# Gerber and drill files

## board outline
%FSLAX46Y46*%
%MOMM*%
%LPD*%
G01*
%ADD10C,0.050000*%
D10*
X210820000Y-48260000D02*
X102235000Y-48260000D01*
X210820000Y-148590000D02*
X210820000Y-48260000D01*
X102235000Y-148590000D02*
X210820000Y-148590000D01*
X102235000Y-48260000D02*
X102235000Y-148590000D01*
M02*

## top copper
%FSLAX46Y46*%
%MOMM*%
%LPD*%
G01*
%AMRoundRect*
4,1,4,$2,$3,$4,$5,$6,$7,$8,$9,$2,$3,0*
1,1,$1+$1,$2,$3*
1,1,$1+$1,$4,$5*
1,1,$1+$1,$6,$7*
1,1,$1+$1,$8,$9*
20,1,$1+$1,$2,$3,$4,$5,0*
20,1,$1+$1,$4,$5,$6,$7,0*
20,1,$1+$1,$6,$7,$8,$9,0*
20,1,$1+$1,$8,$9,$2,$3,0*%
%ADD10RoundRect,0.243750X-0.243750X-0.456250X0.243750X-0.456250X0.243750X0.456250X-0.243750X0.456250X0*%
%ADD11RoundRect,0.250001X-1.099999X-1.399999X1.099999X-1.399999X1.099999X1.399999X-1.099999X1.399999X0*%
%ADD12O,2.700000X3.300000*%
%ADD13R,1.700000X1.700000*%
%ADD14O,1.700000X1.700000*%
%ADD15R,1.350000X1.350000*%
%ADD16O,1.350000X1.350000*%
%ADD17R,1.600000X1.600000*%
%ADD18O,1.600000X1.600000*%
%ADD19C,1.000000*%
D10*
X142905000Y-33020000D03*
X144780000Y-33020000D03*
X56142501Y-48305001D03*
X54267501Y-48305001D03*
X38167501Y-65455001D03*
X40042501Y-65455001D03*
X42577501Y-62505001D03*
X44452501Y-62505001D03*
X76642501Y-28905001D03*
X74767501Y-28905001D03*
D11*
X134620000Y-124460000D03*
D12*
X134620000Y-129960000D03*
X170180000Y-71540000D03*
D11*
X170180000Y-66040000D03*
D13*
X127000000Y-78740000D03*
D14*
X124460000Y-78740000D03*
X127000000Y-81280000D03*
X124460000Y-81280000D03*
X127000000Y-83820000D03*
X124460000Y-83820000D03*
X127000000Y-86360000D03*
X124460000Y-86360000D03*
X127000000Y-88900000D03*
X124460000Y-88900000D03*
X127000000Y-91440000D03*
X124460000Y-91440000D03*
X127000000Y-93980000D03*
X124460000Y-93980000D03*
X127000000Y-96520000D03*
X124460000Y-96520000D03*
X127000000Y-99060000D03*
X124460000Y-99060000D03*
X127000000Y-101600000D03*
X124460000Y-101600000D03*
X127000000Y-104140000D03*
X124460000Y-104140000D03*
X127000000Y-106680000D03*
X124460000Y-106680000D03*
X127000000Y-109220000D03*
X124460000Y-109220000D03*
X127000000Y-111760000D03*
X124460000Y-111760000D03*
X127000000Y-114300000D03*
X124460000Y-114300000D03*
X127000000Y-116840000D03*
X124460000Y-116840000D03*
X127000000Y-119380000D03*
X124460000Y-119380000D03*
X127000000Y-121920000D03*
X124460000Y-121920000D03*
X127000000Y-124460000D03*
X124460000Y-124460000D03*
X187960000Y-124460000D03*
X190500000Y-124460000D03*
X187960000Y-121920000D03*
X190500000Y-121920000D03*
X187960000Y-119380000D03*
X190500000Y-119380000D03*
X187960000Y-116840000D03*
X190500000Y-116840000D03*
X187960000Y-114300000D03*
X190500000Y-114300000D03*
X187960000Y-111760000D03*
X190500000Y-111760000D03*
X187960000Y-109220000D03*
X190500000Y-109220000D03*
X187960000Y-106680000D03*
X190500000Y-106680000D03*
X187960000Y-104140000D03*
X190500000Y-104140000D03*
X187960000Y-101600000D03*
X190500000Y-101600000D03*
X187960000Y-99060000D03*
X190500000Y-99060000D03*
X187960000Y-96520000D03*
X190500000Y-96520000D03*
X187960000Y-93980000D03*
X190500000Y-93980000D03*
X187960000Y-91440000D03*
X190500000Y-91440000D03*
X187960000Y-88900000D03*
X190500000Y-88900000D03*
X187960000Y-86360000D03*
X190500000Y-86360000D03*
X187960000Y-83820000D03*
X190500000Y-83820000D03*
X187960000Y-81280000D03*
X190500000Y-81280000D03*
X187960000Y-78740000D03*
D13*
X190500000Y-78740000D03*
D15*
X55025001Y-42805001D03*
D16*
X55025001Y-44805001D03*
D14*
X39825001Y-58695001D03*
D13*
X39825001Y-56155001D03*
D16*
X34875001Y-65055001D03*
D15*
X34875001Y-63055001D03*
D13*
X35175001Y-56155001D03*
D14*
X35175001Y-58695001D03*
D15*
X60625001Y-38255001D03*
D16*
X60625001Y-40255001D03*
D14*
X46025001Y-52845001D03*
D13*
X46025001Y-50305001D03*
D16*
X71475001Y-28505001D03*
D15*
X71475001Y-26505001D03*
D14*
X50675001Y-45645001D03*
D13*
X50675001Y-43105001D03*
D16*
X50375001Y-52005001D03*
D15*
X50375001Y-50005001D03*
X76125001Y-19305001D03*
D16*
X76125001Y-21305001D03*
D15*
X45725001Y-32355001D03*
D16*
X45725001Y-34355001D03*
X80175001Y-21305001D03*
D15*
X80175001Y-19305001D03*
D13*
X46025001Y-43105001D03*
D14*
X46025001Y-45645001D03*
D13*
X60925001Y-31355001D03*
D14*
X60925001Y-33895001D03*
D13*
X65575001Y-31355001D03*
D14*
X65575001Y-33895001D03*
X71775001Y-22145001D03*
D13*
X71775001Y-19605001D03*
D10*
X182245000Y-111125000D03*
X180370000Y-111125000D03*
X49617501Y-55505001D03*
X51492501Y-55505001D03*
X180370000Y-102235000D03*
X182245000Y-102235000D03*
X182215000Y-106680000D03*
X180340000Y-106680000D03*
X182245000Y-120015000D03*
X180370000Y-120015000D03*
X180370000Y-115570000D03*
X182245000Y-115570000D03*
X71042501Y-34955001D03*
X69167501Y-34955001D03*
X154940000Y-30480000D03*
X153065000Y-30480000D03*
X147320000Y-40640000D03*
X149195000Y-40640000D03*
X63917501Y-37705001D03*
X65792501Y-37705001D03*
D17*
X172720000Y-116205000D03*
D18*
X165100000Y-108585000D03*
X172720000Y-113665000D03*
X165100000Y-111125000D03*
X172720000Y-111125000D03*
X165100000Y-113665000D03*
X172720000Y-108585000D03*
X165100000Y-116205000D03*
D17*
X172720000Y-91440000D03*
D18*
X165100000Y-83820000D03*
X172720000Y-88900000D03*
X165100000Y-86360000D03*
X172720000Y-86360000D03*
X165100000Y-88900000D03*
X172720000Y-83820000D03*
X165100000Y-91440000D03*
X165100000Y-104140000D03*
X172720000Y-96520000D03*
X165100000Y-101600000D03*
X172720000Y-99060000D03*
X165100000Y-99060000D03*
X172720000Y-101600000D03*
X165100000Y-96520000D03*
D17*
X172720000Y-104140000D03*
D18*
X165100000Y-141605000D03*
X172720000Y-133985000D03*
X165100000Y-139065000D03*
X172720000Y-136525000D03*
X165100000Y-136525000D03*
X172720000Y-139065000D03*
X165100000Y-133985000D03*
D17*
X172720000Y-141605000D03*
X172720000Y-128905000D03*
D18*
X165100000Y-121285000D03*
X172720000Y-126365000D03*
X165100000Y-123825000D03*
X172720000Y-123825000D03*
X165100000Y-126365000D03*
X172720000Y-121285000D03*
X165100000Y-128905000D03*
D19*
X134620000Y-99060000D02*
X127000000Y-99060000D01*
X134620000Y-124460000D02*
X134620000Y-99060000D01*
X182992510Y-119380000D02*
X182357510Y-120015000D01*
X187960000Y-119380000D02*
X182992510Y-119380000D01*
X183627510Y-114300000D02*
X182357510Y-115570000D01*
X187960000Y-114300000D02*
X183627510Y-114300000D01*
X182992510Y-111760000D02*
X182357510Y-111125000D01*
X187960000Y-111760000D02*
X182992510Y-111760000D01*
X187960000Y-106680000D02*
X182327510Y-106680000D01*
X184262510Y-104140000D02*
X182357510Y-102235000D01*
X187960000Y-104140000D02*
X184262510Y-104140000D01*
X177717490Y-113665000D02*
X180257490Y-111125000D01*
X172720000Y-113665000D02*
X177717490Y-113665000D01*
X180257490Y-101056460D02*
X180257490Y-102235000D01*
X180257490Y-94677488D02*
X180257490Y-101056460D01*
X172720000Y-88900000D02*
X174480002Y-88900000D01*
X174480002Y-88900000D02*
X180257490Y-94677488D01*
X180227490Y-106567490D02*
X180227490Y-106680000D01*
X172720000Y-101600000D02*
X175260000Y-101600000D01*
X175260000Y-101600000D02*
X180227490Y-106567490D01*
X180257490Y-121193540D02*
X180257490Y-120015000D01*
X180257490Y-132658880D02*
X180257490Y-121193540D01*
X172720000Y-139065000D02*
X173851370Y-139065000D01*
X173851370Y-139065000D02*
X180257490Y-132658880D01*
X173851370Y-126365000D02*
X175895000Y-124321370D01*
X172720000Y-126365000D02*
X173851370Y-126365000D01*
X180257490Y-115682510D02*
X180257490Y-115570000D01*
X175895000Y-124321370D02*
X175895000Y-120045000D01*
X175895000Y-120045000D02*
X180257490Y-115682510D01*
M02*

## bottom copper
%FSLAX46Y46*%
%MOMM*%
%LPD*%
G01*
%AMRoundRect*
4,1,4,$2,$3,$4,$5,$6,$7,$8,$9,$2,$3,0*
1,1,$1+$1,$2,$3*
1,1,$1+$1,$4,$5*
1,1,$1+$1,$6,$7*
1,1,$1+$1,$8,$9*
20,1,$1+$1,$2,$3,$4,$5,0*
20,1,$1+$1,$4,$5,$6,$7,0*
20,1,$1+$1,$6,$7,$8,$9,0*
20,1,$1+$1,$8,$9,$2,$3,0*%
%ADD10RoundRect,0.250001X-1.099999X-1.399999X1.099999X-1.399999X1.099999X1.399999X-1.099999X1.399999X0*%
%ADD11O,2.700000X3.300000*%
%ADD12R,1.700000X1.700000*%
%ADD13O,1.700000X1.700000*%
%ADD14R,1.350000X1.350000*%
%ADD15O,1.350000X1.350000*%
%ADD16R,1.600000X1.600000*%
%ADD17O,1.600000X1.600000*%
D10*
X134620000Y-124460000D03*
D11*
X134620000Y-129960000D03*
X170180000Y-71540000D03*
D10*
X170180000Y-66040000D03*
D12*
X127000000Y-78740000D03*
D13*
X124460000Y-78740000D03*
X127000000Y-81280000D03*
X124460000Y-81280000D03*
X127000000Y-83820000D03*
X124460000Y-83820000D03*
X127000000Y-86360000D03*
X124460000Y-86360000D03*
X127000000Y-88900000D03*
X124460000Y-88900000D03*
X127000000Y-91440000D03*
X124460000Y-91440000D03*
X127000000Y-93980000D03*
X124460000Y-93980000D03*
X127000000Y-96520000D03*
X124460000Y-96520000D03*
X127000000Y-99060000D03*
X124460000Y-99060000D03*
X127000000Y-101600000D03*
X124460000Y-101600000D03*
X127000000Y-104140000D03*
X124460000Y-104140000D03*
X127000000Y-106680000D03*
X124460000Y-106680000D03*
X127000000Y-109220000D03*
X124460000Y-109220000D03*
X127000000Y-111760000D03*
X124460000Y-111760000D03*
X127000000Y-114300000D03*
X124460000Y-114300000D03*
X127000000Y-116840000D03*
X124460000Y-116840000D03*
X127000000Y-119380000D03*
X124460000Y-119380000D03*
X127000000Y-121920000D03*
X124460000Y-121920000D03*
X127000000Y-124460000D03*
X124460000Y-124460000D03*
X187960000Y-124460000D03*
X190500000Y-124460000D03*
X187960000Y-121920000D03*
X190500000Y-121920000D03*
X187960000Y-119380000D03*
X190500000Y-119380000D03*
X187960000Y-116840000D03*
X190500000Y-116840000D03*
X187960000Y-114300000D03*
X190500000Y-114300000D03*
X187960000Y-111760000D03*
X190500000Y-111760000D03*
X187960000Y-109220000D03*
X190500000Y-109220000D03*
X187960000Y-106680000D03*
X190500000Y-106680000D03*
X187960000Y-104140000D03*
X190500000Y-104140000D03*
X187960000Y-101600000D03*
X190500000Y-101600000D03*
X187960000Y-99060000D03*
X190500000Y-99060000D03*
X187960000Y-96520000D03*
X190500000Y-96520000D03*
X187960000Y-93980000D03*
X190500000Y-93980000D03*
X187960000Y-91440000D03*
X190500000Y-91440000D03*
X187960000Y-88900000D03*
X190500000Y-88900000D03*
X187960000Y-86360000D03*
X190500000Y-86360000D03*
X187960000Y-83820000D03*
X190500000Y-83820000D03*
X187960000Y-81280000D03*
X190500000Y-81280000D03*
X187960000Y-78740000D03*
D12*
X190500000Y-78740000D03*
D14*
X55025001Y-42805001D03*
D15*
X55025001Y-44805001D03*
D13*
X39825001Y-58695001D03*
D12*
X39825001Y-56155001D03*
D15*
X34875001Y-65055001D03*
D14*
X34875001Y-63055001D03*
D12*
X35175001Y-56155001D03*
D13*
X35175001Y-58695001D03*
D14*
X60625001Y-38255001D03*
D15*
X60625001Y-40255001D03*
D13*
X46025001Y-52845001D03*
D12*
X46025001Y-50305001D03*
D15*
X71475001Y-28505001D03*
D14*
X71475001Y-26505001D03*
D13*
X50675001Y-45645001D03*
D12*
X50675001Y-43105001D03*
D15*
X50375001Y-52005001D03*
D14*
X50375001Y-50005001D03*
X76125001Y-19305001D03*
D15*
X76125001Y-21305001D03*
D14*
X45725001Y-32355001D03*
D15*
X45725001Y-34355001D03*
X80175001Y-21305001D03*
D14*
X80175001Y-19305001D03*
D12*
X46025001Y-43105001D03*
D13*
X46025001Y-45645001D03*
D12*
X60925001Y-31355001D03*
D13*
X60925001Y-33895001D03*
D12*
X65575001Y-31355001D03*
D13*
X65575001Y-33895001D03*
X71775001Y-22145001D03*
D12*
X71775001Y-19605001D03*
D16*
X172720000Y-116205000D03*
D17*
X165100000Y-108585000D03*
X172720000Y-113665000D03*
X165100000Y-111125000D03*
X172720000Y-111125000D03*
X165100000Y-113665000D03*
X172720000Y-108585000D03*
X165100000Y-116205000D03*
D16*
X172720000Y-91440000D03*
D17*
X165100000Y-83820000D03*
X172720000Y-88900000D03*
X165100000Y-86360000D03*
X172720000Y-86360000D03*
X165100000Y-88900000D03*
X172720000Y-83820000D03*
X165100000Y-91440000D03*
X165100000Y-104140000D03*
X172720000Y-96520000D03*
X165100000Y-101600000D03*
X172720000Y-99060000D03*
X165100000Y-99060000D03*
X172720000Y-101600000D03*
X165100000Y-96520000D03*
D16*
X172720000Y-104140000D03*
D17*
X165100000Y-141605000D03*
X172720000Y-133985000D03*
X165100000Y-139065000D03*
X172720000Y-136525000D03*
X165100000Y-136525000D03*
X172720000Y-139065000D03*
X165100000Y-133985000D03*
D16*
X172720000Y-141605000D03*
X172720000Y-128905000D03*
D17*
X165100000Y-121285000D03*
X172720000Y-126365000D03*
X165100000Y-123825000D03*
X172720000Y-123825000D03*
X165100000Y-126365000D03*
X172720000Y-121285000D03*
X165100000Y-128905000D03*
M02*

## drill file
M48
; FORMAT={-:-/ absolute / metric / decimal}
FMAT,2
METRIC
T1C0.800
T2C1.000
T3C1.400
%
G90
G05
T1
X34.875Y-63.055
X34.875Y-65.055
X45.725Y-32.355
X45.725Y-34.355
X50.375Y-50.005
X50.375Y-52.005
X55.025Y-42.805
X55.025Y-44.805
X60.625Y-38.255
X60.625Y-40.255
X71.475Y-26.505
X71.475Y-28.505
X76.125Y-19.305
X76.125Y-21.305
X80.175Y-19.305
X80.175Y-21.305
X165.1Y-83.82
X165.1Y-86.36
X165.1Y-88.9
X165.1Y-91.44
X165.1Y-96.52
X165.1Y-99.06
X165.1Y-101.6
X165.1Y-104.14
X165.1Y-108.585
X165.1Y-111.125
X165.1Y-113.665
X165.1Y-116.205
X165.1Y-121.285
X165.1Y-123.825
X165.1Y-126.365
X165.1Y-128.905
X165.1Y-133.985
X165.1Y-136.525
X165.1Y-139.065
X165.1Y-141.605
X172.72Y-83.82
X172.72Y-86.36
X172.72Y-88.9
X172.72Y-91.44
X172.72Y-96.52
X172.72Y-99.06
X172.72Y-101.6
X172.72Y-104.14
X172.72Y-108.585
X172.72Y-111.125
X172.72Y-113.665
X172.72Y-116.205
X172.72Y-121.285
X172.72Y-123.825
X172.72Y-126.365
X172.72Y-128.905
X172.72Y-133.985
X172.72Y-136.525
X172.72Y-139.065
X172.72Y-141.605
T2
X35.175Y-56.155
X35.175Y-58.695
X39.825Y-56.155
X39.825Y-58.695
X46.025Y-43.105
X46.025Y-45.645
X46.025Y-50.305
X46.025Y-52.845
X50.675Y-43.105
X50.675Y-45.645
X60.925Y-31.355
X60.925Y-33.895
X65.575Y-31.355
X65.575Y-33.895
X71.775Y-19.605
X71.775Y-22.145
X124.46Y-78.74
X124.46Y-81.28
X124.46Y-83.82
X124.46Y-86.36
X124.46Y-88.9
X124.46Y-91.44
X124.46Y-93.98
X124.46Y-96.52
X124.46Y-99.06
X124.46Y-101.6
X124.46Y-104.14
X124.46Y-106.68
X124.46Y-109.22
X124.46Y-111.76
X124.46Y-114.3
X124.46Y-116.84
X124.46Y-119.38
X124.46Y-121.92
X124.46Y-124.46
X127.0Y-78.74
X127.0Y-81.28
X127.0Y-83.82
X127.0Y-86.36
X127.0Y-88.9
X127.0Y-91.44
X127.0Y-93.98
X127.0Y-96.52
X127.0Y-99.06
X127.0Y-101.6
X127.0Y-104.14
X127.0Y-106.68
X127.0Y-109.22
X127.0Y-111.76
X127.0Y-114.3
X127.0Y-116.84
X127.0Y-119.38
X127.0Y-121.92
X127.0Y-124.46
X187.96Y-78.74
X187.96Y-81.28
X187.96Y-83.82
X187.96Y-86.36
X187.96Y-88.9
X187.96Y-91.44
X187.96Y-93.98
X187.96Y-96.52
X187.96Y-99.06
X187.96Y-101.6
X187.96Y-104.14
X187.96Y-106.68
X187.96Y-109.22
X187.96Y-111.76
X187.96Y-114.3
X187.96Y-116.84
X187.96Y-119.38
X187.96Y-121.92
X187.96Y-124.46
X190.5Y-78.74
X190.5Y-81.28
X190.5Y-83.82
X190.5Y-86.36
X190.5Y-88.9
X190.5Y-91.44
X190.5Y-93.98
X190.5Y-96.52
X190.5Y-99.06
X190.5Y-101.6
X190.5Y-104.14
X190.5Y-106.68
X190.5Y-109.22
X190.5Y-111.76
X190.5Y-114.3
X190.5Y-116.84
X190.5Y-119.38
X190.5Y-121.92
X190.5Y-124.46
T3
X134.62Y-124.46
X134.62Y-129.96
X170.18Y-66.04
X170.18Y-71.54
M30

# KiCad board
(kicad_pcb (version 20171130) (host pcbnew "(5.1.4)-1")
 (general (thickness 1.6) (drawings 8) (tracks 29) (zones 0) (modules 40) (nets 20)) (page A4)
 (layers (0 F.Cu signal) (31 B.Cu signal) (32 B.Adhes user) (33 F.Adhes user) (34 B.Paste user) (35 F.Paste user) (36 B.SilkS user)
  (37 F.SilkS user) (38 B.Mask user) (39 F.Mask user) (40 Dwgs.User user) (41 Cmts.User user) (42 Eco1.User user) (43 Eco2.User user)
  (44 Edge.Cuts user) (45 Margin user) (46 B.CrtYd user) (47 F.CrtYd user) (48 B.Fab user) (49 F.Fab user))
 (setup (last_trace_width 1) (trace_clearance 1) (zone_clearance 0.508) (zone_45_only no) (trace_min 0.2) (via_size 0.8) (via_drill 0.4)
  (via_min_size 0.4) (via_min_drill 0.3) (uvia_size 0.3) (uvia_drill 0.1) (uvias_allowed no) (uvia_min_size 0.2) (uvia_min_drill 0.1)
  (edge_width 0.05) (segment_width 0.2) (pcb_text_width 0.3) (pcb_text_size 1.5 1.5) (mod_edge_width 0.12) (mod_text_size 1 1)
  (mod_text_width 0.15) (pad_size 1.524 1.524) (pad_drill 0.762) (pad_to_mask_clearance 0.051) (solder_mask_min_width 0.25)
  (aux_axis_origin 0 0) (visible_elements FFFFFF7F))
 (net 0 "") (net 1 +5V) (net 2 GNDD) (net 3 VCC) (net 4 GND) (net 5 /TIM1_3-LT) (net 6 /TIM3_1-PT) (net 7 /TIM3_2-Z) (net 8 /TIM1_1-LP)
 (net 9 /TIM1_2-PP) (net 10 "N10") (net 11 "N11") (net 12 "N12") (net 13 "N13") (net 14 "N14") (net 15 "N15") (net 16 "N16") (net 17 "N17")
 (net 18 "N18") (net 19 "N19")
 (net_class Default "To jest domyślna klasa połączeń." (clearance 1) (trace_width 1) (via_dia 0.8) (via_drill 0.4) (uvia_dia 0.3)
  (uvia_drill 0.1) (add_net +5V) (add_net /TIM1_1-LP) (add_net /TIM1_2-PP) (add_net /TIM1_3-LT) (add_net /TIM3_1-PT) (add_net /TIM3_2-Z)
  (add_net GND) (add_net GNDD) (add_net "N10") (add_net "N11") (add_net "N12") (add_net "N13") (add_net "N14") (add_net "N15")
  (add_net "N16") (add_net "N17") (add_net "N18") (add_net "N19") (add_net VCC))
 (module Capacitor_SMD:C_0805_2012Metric (layer F.Cu) (at 143.8425 33.02)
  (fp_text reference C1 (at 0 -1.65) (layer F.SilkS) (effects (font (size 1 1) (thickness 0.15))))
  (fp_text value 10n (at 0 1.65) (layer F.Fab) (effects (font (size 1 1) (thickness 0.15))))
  (pad 1 smd roundrect (at -0.9375 0) (size 0.975 1.4) (layers F.Cu F.Paste F.Mask) (roundrect_rratio 0.25) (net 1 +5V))
  (pad 2 smd roundrect (at 0.9375 0) (size 0.975 1.4) (layers F.Cu F.Paste F.Mask) (roundrect_rratio 0.25) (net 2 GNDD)))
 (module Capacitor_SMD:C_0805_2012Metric (layer F.Cu) (at 55.205001 48.305001)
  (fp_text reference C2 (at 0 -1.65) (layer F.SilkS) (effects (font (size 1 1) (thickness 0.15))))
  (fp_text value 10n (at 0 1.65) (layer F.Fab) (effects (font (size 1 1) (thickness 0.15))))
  (pad 2 smd roundrect (at 0.9375 0) (size 0.975 1.4) (layers F.Cu F.Paste F.Mask) (roundrect_rratio 0.25) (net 2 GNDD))
  (pad 1 smd roundrect (at -0.9375 0) (size 0.975 1.4) (layers F.Cu F.Paste F.Mask) (roundrect_rratio 0.25) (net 1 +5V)))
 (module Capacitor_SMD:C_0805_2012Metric (layer F.Cu) (at 39.105001 65.455001)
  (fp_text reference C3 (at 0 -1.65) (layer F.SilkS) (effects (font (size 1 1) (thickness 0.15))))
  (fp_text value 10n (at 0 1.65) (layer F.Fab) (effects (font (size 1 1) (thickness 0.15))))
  (pad 1 smd roundrect (at -0.9375 0) (size 0.975 1.4) (layers F.Cu F.Paste F.Mask) (roundrect_rratio 0.25) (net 1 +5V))
  (pad 2 smd roundrect (at 0.9375 0) (size 0.975 1.4) (layers F.Cu F.Paste F.Mask) (roundrect_rratio 0.25) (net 2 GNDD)))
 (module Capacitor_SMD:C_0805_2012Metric (layer F.Cu) (at 43.515001 62.505001)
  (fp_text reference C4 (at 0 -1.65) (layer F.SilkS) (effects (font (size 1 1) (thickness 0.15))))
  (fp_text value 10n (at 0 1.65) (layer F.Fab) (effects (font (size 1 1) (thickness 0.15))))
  (pad 1 smd roundrect (at -0.9375 0) (size 0.975 1.4) (layers F.Cu F.Paste F.Mask) (roundrect_rratio 0.25) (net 1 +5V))
  (pad 2 smd roundrect (at 0.9375 0) (size 0.975 1.4) (layers F.Cu F.Paste F.Mask) (roundrect_rratio 0.25) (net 2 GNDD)))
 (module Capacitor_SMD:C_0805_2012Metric (layer F.Cu) (at 75.705001 28.905001)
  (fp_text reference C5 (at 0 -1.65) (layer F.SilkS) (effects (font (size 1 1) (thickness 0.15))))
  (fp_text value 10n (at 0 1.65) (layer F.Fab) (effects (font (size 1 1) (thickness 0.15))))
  (pad 2 smd roundrect (at 0.9375 0) (size 0.975 1.4) (layers F.Cu F.Paste F.Mask) (roundrect_rratio 0.25) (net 2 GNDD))
  (pad 1 smd roundrect (at -0.9375 0) (size 0.975 1.4) (layers F.Cu F.Paste F.Mask) (roundrect_rratio 0.25) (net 1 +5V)))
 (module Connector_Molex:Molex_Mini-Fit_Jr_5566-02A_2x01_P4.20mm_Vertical (layer F.Cu) (at 134.62 124.46)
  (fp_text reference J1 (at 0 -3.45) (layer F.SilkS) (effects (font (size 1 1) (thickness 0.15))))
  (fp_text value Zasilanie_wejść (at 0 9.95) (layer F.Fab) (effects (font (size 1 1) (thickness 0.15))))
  (pad 1 thru_hole roundrect (at 0 0) (size 2.7 3.3) (drill 1.4) (layers *.Cu *.Mask) (roundrect_rratio 0.09259299999999999) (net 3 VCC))
  (pad 2 thru_hole oval (at 0 5.5) (size 2.7 3.3) (drill 1.4) (layers *.Cu *.Mask) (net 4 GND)))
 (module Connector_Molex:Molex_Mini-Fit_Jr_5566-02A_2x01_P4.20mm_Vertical (layer F.Cu) (at 170.18 66.04)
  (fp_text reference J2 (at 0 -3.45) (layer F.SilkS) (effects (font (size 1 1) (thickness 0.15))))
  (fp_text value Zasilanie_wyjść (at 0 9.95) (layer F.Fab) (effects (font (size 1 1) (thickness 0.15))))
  (pad 2 thru_hole oval (at 0 5.5) (size 2.7 3.3) (drill 1.4) (layers *.Cu *.Mask) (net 2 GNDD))
  (pad 1 thru_hole roundrect (at 0 0) (size 2.7 3.3) (drill 1.4) (layers *.Cu *.Mask) (roundrect_rratio 0.09259299999999999) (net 1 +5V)))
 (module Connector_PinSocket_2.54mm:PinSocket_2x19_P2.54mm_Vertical (layer F.Cu) (at 127 78.74)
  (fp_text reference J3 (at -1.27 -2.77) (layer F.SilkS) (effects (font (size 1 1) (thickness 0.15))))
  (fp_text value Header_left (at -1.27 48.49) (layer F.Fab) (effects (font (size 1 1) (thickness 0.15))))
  (pad 1 thru_hole rect (at 0 0) (size 1.7 1.7) (drill 1) (layers *.Cu *.Mask))
  (pad 2 thru_hole oval (at -2.54 0) (size 1.7 1.7) (drill 1) (layers *.Cu *.Mask))
  (pad 3 thru_hole oval (at 0 2.54) (size 1.7 1.7) (drill 1) (layers *.Cu *.Mask))
  (pad 4 thru_hole oval (at -2.54 2.54) (size 1.7 1.7) (drill 1) (layers *.Cu *.Mask))
  (pad 5 thru_hole oval (at 0 5.08) (size 1.7 1.7) (drill 1) (layers *.Cu *.Mask))
  (pad 6 thru_hole oval (at -2.54 5.08) (size 1.7 1.7) (drill 1) (layers *.Cu *.Mask))
  (pad 7 thru_hole oval (at 0 7.62) (size 1.7 1.7) (drill 1) (layers *.Cu *.Mask))
  (pad 8 thru_hole oval (at -2.54 7.62) (size 1.7 1.7) (drill 1) (layers *.Cu *.Mask))
  (pad 9 thru_hole oval (at 0 10.16) (size 1.7 1.7) (drill 1) (layers *.Cu *.Mask))
  (pad 10 thru_hole oval (at -2.54 10.16) (size 1.7 1.7) (drill 1) (layers *.Cu *.Mask))
  (pad 11 thru_hole oval (at 0 12.7) (size 1.7 1.7) (drill 1) (layers *.Cu *.Mask))
  (pad 12 thru_hole oval (at -2.54 12.7) (size 1.7 1.7) (drill 1) (layers *.Cu *.Mask))
  (pad 13 thru_hole oval (at 0 15.24) (size 1.7 1.7) (drill 1) (layers *.Cu *.Mask))
  (pad 14 thru_hole oval (at -2.54 15.24) (size 1.7 1.7) (drill 1) (layers *.Cu *.Mask))
  (pad 15 thru_hole oval (at 0 17.78) (size 1.7 1.7) (drill 1) (layers *.Cu *.Mask))
  (pad 16 thru_hole oval (at -2.54 17.78) (size 1.7 1.7) (drill 1) (layers *.Cu *.Mask))
  (pad 17 thru_hole oval (at 0 20.32) (size 1.7 1.7) (drill 1) (layers *.Cu *.Mask) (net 3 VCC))
  (pad 18 thru_hole oval (at -2.54 20.32) (size 1.7 1.7) (drill 1) (layers *.Cu *.Mask))
  (pad 19 thru_hole oval (at 0 22.86) (size 1.7 1.7) (drill 1) (layers *.Cu *.Mask) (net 4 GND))
  (pad 20 thru_hole oval (at -2.54 22.86) (size 1.7 1.7) (drill 1) (layers *.Cu *.Mask))
  (pad 21 thru_hole oval (at 0 25.4) (size 1.7 1.7) (drill 1) (layers *.Cu *.Mask))
  (pad 22 thru_hole oval (at -2.54 25.4) (size 1.7 1.7) (drill 1) (layers *.Cu *.Mask))
  (pad 23 thru_hole oval (at 0 27.94) (size 1.7 1.7) (drill 1) (layers *.Cu *.Mask))
  (pad 24 thru_hole oval (at -2.54 27.94) (size 1.7 1.7) (drill 1) (layers *.Cu *.Mask))
  (pad 25 thru_hole oval (at 0 30.48) (size 1.7 1.7) (drill 1) (layers *.Cu *.Mask))
  (pad 26 thru_hole oval (at -2.54 30.48) (size 1.7 1.7) (drill 1) (layers *.Cu *.Mask))
  (pad 27 thru_hole oval (at 0 33.02) (size 1.7 1.7) (drill 1) (layers *.Cu *.Mask))
  (pad 28 thru_hole oval (at -2.54 33.02) (size 1.7 1.7) (drill 1) (layers *.Cu *.Mask))
  (pad 29 thru_hole oval (at 0 35.56) (size 1.7 1.7) (drill 1) (layers *.Cu *.Mask))
  (pad 30 thru_hole oval (at -2.54 35.56) (size 1.7 1.7) (drill 1) (layers *.Cu *.Mask))
  (pad 31 thru_hole oval (at 0 38.1) (size 1.7 1.7) (drill 1) (layers *.Cu *.Mask))
  (pad 32 thru_hole oval (at -2.54 38.1) (size 1.7 1.7) (drill 1) (layers *.Cu *.Mask))
  (pad 33 thru_hole oval (at 0 40.64) (size 1.7 1.7) (drill 1) (layers *.Cu *.Mask))
  (pad 34 thru_hole oval (at -2.54 40.64) (size 1.7 1.7) (drill 1) (layers *.Cu *.Mask))
  (pad 35 thru_hole oval (at 0 43.18) (size 1.7 1.7) (drill 1) (layers *.Cu *.Mask))
  (pad 36 thru_hole oval (at -2.54 43.18) (size 1.7 1.7) (drill 1) (layers *.Cu *.Mask))
  (pad 37 thru_hole oval (at 0 45.72) (size 1.7 1.7) (drill 1) (layers *.Cu *.Mask))
  (pad 38 thru_hole oval (at -2.54 45.72) (size 1.7 1.7) (drill 1) (layers *.Cu *.Mask)))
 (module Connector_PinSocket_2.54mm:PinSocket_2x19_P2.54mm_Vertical (layer F.Cu) (at 190.5 78.74)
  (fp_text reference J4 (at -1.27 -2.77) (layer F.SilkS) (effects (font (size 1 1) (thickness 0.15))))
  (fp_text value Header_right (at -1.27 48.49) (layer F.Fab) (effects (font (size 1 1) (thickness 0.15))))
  (pad 38 thru_hole oval (at -2.54 45.72) (size 1.7 1.7) (drill 1) (layers *.Cu *.Mask))
  (pad 37 thru_hole oval (at 0 45.72) (size 1.7 1.7) (drill 1) (layers *.Cu *.Mask))
  (pad 36 thru_hole oval (at -2.54 43.18) (size 1.7 1.7) (drill 1) (layers *.Cu *.Mask))
  (pad 35 thru_hole oval (at 0 43.18) (size 1.7 1.7) (drill 1) (layers *.Cu *.Mask))
  (pad 34 thru_hole oval (at -2.54 40.64) (size 1.7 1.7) (drill 1) (layers *.Cu *.Mask) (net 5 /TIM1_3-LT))
  (pad 33 thru_hole oval (at 0 40.64) (size 1.7 1.7) (drill 1) (layers *.Cu *.Mask))
  (pad 32 thru_hole oval (at -2.54 38.1) (size 1.7 1.7) (drill 1) (layers *.Cu *.Mask))
  (pad 31 thru_hole oval (at 0 38.1) (size 1.7 1.7) (drill 1) (layers *.Cu *.Mask))
  (pad 30 thru_hole oval (at -2.54 35.56) (size 1.7 1.7) (drill 1) (layers *.Cu *.Mask) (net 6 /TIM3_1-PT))
  (pad 29 thru_hole oval (at 0 35.56) (size 1.7 1.7) (drill 1) (layers *.Cu *.Mask))
  (pad 28 thru_hole oval (at -2.54 33.02) (size 1.7 1.7) (drill 1) (layers *.Cu *.Mask) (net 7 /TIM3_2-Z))
  (pad 27 thru_hole oval (at 0 33.02) (size 1.7 1.7) (drill 1) (layers *.Cu *.Mask))
  (pad 26 thru_hole oval (at -2.54 30.48) (size 1.7 1.7) (drill 1) (layers *.Cu *.Mask))
  (pad 25 thru_hole oval (at 0 30.48) (size 1.7 1.7) (drill 1) (layers *.Cu *.Mask))
  (pad 24 thru_hole oval (at -2.54 27.94) (size 1.7 1.7) (drill 1) (layers *.Cu *.Mask) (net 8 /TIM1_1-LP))
  (pad 23 thru_hole oval (at 0 27.94) (size 1.7 1.7) (drill 1) (layers *.Cu *.Mask))
  (pad 22 thru_hole oval (at -2.54 25.4) (size 1.7 1.7) (drill 1) (layers *.Cu *.Mask) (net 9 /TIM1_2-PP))
  (pad 21 thru_hole oval (at 0 25.4) (size 1.7 1.7) (drill 1) (layers *.Cu *.Mask))
  (pad 20 thru_hole oval (at -2.54 22.86) (size 1.7 1.7) (drill 1) (layers *.Cu *.Mask))
  (pad 19 thru_hole oval (at 0 22.86) (size 1.7 1.7) (drill 1) (layers *.Cu *.Mask))
  (pad 18 thru_hole oval (at -2.54 20.32) (size 1.7 1.7) (drill 1) (layers *.Cu *.Mask))
  (pad 17 thru_hole oval (at 0 20.32) (size 1.7 1.7) (drill 1) (layers *.Cu *.Mask))
  (pad 16 thru_hole oval (at -2.54 17.78) (size 1.7 1.7) (drill 1) (layers *.Cu *.Mask))
  (pad 15 thru_hole oval (at 0 17.78) (size 1.7 1.7) (drill 1) (layers *.Cu *.Mask))
  (pad 14 thru_hole oval (at -2.54 15.24) (size 1.7 1.7) (drill 1) (layers *.Cu *.Mask))
  (pad 13 thru_hole oval (at 0 15.24) (size 1.7 1.7) (drill 1) (layers *.Cu *.Mask))
  (pad 12 thru_hole oval (at -2.54 12.7) (size 1.7 1.7) (drill 1) (layers *.Cu *.Mask))
  (pad 11 thru_hole oval (at 0 12.7) (size 1.7 1.7) (drill 1) (layers *.Cu *.Mask))
  (pad 10 thru_hole oval (at -2.54 10.16) (size 1.7 1.7) (drill 1) (layers *.Cu *.Mask))
  (pad 9 thru_hole oval (at 0 10.16) (size 1.7 1.7) (drill 1) (layers *.Cu *.Mask))
  (pad 8 thru_hole oval (at -2.54 7.62) (size 1.7 1.7) (drill 1) (layers *.Cu *.Mask))
  (pad 7 thru_hole oval (at 0 7.62) (size 1.7 1.7) (drill 1) (layers *.Cu *.Mask))
  (pad 6 thru_hole oval (at -2.54 5.08) (size 1.7 1.7) (drill 1) (layers *.Cu *.Mask))
  (pad 5 thru_hole oval (at 0 5.08) (size 1.7 1.7) (drill 1) (layers *.Cu *.Mask))
  (pad 4 thru_hole oval (at -2.54 2.54) (size 1.7 1.7) (drill 1) (layers *.Cu *.Mask))
  (pad 3 thru_hole oval (at 0 2.54) (size 1.7 1.7) (drill 1) (layers *.Cu *.Mask))
  (pad 2 thru_hole oval (at -2.54 0) (size 1.7 1.7) (drill 1) (layers *.Cu *.Mask))
  (pad 1 thru_hole rect (at 0 0) (size 1.7 1.7) (drill 1) (layers *.Cu *.Mask)))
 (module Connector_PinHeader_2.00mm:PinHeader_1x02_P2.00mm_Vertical (layer F.Cu) (at 55.025001 42.805001)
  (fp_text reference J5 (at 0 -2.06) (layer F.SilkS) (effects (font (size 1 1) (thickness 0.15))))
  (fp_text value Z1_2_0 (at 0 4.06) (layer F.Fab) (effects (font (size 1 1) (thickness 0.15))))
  (pad 1 thru_hole rect (at 0 0) (size 1.35 1.35) (drill 0.8) (layers *.Cu *.Mask) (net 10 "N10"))
  (pad 2 thru_hole oval (at 0 2) (size 1.35 1.35) (drill 0.8) (layers *.Cu *.Mask) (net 2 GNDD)))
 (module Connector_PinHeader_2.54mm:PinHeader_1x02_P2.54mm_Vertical (layer F.Cu) (at 39.825001 56.155001)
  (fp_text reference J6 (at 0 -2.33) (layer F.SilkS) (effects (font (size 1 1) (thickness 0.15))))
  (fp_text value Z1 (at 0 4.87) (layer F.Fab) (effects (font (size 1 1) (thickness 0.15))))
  (pad 2 thru_hole oval (at 0 2.54) (size 1.7 1.7) (drill 1) (layers *.Cu *.Mask) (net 2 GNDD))
  (pad 1 thru_hole rect (at 0 0) (size 1.7 1.7) (drill 1) (layers *.Cu *.Mask) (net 10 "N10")))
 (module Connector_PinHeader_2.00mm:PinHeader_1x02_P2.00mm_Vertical (layer F.Cu) (at 34.875001 63.055001)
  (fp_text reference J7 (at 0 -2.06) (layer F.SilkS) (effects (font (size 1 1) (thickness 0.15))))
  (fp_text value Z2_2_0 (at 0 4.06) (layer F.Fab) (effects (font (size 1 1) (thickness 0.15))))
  (pad 2 thru_hole oval (at 0 2) (size 1.35 1.35) (drill 0.8) (layers *.Cu *.Mask) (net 2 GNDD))
  (pad 1 thru_hole rect (at 0 0) (size 1.35 1.35) (drill 0.8) (layers *.Cu *.Mask) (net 10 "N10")))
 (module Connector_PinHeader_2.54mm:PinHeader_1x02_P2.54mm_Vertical (layer F.Cu) (at 35.175001 56.155001)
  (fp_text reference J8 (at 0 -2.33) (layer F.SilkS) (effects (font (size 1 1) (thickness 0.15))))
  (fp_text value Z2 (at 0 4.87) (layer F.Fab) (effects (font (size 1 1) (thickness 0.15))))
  (pad 1 thru_hole rect (at 0 0) (size 1.7 1.7) (drill 1) (layers *.Cu *.Mask) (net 10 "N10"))
  (pad 2 thru_hole oval (at 0 2.54) (size 1.7 1.7) (drill 1) (layers *.Cu *.Mask) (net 2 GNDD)))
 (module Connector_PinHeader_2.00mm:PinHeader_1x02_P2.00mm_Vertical (layer F.Cu) (at 60.625001 38.255001)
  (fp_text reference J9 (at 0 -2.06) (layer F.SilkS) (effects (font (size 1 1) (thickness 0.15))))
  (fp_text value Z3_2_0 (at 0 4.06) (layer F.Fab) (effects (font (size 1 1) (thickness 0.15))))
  (pad 1 thru_hole rect (at 0 0) (size 1.35 1.35) (drill 0.8) (layers *.Cu *.Mask) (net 10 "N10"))
  (pad 2 thru_hole oval (at 0 2) (size 1.35 1.35) (drill 0.8) (layers *.Cu *.Mask) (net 2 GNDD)))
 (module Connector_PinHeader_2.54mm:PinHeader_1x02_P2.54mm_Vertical (layer F.Cu) (at 46.025001 50.305001)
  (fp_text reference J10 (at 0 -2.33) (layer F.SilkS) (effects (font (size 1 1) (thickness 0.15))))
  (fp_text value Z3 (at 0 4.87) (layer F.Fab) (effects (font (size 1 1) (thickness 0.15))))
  (pad 2 thru_hole oval (at 0 2.54) (size 1.7 1.7) (drill 1) (layers *.Cu *.Mask) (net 2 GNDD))
  (pad 1 thru_hole rect (at 0 0) (size 1.7 1.7) (drill 1) (layers *.Cu *.Mask) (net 10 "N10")))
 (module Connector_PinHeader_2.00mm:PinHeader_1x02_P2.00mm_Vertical (layer F.Cu) (at 71.475001 26.505001)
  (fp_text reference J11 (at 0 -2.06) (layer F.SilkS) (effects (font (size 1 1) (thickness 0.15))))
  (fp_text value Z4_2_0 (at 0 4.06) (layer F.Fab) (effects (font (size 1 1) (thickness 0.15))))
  (pad 2 thru_hole oval (at 0 2) (size 1.35 1.35) (drill 0.8) (layers *.Cu *.Mask) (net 2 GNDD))
  (pad 1 thru_hole rect (at 0 0) (size 1.35 1.35) (drill 0.8) (layers *.Cu *.Mask) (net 10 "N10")))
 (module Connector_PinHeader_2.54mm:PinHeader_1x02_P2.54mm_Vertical (layer F.Cu) (at 50.675001 43.105001)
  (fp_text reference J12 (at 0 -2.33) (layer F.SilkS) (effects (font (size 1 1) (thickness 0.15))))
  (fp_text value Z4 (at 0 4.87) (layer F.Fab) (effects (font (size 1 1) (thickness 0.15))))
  (pad 2 thru_hole oval (at 0 2.54) (size 1.7 1.7) (drill 1) (layers *.Cu *.Mask) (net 2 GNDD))
  (pad 1 thru_hole rect (at 0 0) (size 1.7 1.7) (drill 1) (layers *.Cu *.Mask) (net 10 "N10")))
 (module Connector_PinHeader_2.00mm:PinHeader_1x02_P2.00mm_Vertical (layer F.Cu) (at 50.375001 50.005001)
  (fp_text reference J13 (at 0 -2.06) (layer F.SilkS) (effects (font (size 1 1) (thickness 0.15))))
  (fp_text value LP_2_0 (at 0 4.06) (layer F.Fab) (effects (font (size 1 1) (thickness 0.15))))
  (pad 2 thru_hole oval (at 0 2) (size 1.35 1.35) (drill 0.8) (layers *.Cu *.Mask) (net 2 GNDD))
  (pad 1 thru_hole rect (at 0 0) (size 1.35 1.35) (drill 0.8) (layers *.Cu *.Mask) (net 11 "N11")))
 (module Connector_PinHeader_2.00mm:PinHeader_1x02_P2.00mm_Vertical (layer F.Cu) (at 76.125001 19.305001)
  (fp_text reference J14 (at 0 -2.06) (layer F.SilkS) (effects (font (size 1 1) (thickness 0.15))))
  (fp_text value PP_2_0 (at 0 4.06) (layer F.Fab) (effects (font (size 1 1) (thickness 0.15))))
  (pad 1 thru_hole rect (at 0 0) (size 1.35 1.35) (drill 0.8) (layers *.Cu *.Mask) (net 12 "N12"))
  (pad 2 thru_hole oval (at 0 2) (size 1.35 1.35) (drill 0.8) (layers *.Cu *.Mask) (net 2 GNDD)))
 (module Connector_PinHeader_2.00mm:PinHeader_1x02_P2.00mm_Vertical (layer F.Cu) (at 45.725001 32.355001)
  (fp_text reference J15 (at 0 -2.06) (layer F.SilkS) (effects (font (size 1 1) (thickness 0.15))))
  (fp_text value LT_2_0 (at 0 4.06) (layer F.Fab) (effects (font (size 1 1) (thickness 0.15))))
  (pad 1 thru_hole rect (at 0 0) (size 1.35 1.35) (drill 0.8) (layers *.Cu *.Mask) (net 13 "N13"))
  (pad 2 thru_hole oval (at 0 2) (size 1.35 1.35) (drill 0.8) (layers *.Cu *.Mask) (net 2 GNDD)))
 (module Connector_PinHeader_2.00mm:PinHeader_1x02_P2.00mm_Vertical (layer F.Cu) (at 80.175001 19.305001)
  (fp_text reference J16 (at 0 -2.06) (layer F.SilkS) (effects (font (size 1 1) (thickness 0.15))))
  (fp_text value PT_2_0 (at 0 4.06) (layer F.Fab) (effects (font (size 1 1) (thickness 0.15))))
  (pad 2 thru_hole oval (at 0 2) (size 1.35 1.35) (drill 0.8) (layers *.Cu *.Mask) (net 2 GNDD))
  (pad 1 thru_hole rect (at 0 0) (size 1.35 1.35) (drill 0.8) (layers *.Cu *.Mask) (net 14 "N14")))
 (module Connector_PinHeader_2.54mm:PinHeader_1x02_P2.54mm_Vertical (layer F.Cu) (at 46.025001 43.105001)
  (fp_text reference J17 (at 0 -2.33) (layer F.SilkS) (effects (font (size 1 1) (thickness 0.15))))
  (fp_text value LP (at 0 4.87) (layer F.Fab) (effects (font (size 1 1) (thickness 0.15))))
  (pad 1 thru_hole rect (at 0 0) (size 1.7 1.7) (drill 1) (layers *.Cu *.Mask) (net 11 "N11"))
  (pad 2 thru_hole oval (at 0 2.54) (size 1.7 1.7) (drill 1) (layers *.Cu *.Mask) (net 2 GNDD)))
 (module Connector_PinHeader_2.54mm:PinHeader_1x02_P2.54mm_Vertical (layer F.Cu) (at 60.925001 31.355001)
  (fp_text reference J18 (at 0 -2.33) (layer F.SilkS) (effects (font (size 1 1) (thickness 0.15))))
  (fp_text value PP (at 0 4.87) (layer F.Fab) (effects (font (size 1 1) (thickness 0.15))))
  (pad 1 thru_hole rect (at 0 0) (size 1.7 1.7) (drill 1) (layers *.Cu *.Mask) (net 12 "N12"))
  (pad 2 thru_hole oval (at 0 2.54) (size 1.7 1.7) (drill 1) (layers *.Cu *.Mask) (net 2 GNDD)))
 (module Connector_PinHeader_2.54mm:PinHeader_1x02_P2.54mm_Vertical (layer F.Cu) (at 65.575001 31.355001)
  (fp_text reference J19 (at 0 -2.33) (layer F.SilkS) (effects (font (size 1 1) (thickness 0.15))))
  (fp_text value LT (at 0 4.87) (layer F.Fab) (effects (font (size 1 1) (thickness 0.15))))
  (pad 1 thru_hole rect (at 0 0) (size 1.7 1.7) (drill 1) (layers *.Cu *.Mask) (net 13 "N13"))
  (pad 2 thru_hole oval (at 0 2.54) (size 1.7 1.7) (drill 1) (layers *.Cu *.Mask) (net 2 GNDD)))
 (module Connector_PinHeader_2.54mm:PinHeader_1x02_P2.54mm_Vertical (layer F.Cu) (at 71.775001 19.605001)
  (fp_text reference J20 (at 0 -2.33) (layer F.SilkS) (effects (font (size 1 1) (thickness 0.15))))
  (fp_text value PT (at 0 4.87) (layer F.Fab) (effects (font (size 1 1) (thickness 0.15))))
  (pad 2 thru_hole oval (at 0 2.54) (size 1.7 1.7) (drill 1) (layers *.Cu *.Mask) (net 2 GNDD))
  (pad 1 thru_hole rect (at 0 0) (size 1.7 1.7) (drill 1) (layers *.Cu *.Mask) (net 14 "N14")))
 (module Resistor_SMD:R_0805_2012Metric (layer F.Cu) (at 181.3075 111.125)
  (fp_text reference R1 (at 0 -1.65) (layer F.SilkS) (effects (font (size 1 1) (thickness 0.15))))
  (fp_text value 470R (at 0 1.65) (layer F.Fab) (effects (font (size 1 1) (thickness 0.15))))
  (pad 2 smd roundrect (at 0.9375 0) (size 0.975 1.4) (layers F.Cu F.Paste F.Mask) (roundrect_rratio 0.25) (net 7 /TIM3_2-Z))
  (pad 1 smd roundrect (at -0.9375 0) (size 0.975 1.4) (layers F.Cu F.Paste F.Mask) (roundrect_rratio 0.25) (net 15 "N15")))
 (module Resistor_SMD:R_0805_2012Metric (layer F.Cu) (at 50.555001 55.505001)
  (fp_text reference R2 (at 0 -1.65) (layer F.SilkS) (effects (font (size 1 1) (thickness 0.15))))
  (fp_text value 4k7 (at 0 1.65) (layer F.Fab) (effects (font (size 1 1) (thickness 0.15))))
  (pad 1 smd roundrect (at -0.9375 0) (size 0.975 1.4) (layers F.Cu F.Paste F.Mask) (roundrect_rratio 0.25) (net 1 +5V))
  (pad 2 smd roundrect (at 0.9375 0) (size 0.975 1.4) (layers F.Cu F.Paste F.Mask) (roundrect_rratio 0.25) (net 10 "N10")))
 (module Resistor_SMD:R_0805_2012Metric (layer F.Cu) (at 181.3075 102.235)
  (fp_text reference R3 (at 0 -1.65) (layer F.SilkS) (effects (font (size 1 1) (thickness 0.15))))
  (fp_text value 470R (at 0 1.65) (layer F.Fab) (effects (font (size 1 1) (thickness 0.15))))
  (pad 1 smd roundrect (at -0.9375 0) (size 0.975 1.4) (layers F.Cu F.Paste F.Mask) (roundrect_rratio 0.25) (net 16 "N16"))
  (pad 2 smd roundrect (at 0.9375 0) (size 0.975 1.4) (layers F.Cu F.Paste F.Mask) (roundrect_rratio 0.25) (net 9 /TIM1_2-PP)))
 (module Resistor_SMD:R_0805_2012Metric (layer F.Cu) (at 181.2775 106.68)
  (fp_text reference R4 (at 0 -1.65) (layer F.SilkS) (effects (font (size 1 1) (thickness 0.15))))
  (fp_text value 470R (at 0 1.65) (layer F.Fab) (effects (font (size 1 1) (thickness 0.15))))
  (pad 2 smd roundrect (at 0.9375 0) (size 0.975 1.4) (layers F.Cu F.Paste F.Mask) (roundrect_rratio 0.25) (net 8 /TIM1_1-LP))
  (pad 1 smd roundrect (at -0.9375 0) (size 0.975 1.4) (layers F.Cu F.Paste F.Mask) (roundrect_rratio 0.25) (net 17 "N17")))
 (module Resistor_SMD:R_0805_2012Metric (layer F.Cu) (at 181.3075 120.015)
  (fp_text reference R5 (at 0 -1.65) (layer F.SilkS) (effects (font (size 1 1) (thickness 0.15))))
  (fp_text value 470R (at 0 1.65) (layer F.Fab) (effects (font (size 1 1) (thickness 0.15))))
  (pad 2 smd roundrect (at 0.9375 0) (size 0.975 1.4) (layers F.Cu F.Paste F.Mask) (roundrect_rratio 0.25) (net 5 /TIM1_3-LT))
  (pad 1 smd roundrect (at -0.9375 0) (size 0.975 1.4) (layers F.Cu F.Paste F.Mask) (roundrect_rratio 0.25) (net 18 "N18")))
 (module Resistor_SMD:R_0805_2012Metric (layer F.Cu) (at 181.3075 115.57)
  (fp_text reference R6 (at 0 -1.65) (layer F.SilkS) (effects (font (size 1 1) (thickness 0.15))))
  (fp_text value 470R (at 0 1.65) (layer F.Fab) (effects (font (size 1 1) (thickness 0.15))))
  (pad 1 smd roundrect (at -0.9375 0) (size 0.975 1.4) (layers F.Cu F.Paste F.Mask) (roundrect_rratio 0.25) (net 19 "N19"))
  (pad 2 smd roundrect (at 0.9375 0) (size 0.975 1.4) (layers F.Cu F.Paste F.Mask) (roundrect_rratio 0.25) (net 6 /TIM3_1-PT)))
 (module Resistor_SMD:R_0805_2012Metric (layer F.Cu) (at 70.105001 34.955001)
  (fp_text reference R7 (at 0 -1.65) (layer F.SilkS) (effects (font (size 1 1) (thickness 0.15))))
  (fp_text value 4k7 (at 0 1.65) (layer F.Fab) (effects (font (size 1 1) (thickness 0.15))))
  (pad 2 smd roundrect (at 0.9375 0) (size 0.975 1.4) (layers F.Cu F.Paste F.Mask) (roundrect_rratio 0.25) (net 12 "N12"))
  (pad 1 smd roundrect (at -0.9375 0) (size 0.975 1.4) (layers F.Cu F.Paste F.Mask) (roundrect_rratio 0.25) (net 1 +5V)))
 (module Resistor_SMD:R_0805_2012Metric (layer F.Cu) (at 154.0025 30.48)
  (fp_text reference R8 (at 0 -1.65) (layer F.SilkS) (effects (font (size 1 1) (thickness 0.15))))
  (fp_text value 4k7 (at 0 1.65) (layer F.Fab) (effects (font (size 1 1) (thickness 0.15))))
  (pad 2 smd roundrect (at 0.9375 0) (size 0.975 1.4) (layers F.Cu F.Paste F.Mask) (roundrect_rratio 0.25) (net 11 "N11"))
  (pad 1 smd roundrect (at -0.9375 0) (size 0.975 1.4) (layers F.Cu F.Paste F.Mask) (roundrect_rratio 0.25) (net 1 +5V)))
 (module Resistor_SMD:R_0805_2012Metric (layer F.Cu) (at 148.2575 40.64)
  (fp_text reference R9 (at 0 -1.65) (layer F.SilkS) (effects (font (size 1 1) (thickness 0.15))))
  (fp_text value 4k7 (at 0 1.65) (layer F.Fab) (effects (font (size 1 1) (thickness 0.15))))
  (pad 1 smd roundrect (at -0.9375 0) (size 0.975 1.4) (layers F.Cu F.Paste F.Mask) (roundrect_rratio 0.25) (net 1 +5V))
  (pad 2 smd roundrect (at 0.9375 0) (size 0.975 1.4) (layers F.Cu F.Paste F.Mask) (roundrect_rratio 0.25) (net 13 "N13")))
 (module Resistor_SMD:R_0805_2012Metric (layer F.Cu) (at 64.855001 37.705001)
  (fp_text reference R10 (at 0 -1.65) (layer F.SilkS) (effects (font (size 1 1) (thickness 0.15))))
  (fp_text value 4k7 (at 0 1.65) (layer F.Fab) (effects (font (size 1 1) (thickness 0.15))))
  (pad 1 smd roundrect (at -0.9375 0) (size 0.975 1.4) (layers F.Cu F.Paste F.Mask) (roundrect_rratio 0.25) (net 1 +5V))
  (pad 2 smd roundrect (at 0.9375 0) (size 0.975 1.4) (layers F.Cu F.Paste F.Mask) (roundrect_rratio 0.25) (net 14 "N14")))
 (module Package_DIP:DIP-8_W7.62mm (layer F.Cu) (at 172.72 116.205 180)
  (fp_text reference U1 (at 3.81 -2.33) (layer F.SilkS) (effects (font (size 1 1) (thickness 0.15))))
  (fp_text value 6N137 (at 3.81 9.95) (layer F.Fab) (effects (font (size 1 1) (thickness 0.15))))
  (pad 1 thru_hole rect (at 0 0 180) (size 1.6 1.6) (drill 0.8) (layers *.Cu *.Mask))
  (pad 5 thru_hole oval (at 7.62 7.62 180) (size 1.6 1.6) (drill 0.8) (layers *.Cu *.Mask) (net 2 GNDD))
  (pad 2 thru_hole oval (at 0 2.54 180) (size 1.6 1.6) (drill 0.8) (layers *.Cu *.Mask) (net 15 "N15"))
  (pad 6 thru_hole oval (at 7.62 5.08 180) (size 1.6 1.6) (drill 0.8) (layers *.Cu *.Mask) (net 10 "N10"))
  (pad 3 thru_hole oval (at 0 5.08 180) (size 1.6 1.6) (drill 0.8) (layers *.Cu *.Mask) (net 4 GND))
  (pad 7 thru_hole oval (at 7.62 2.54 180) (size 1.6 1.6) (drill 0.8) (layers *.Cu *.Mask) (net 1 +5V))
  (pad 4 thru_hole oval (at 0 7.62 180) (size 1.6 1.6) (drill 0.8) (layers *.Cu *.Mask))
  (pad 8 thru_hole oval (at 7.62 0 180) (size 1.6 1.6) (drill 0.8) (layers *.Cu *.Mask) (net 1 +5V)))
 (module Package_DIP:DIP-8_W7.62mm (layer F.Cu) (at 172.72 91.44 180)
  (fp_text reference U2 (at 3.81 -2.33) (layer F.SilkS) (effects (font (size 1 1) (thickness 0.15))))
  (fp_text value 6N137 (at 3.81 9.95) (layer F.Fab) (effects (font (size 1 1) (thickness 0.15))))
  (pad 1 thru_hole rect (at 0 0 180) (size 1.6 1.6) (drill 0.8) (layers *.Cu *.Mask))
  (pad 5 thru_hole oval (at 7.62 7.62 180) (size 1.6 1.6) (drill 0.8) (layers *.Cu *.Mask) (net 2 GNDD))
  (pad 2 thru_hole oval (at 0 2.54 180) (size 1.6 1.6) (drill 0.8) (layers *.Cu *.Mask) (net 16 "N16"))
  (pad 6 thru_hole oval (at 7.62 5.08 180) (size 1.6 1.6) (drill 0.8) (layers *.Cu *.Mask) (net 12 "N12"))
  (pad 3 thru_hole oval (at 0 5.08 180) (size 1.6 1.6) (drill 0.8) (layers *.Cu *.Mask) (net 4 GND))
  (pad 7 thru_hole oval (at 7.62 2.54 180) (size 1.6 1.6) (drill 0.8) (layers *.Cu *.Mask) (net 1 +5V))
  (pad 4 thru_hole oval (at 0 7.62 180) (size 1.6 1.6) (drill 0.8) (layers *.Cu *.Mask))
  (pad 8 thru_hole oval (at 7.62 0 180) (size 1.6 1.6) (drill 0.8) (layers *.Cu *.Mask) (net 1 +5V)))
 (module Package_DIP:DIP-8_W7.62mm (layer F.Cu) (at 172.72 104.14 180)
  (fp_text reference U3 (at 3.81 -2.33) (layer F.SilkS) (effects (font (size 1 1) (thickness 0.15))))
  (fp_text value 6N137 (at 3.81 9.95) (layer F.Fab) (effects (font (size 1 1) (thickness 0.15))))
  (pad 8 thru_hole oval (at 7.62 0 180) (size 1.6 1.6) (drill 0.8) (layers *.Cu *.Mask) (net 1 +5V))
  (pad 4 thru_hole oval (at 0 7.62 180) (size 1.6 1.6) (drill 0.8) (layers *.Cu *.Mask))
  (pad 7 thru_hole oval (at 7.62 2.54 180) (size 1.6 1.6) (drill 0.8) (layers *.Cu *.Mask) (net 1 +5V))
  (pad 3 thru_hole oval (at 0 5.08 180) (size 1.6 1.6) (drill 0.8) (layers *.Cu *.Mask) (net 4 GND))
  (pad 6 thru_hole oval (at 7.62 5.08 180) (size 1.6 1.6) (drill 0.8) (layers *.Cu *.Mask) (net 11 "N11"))
  (pad 2 thru_hole oval (at 0 2.54 180) (size 1.6 1.6) (drill 0.8) (layers *.Cu *.Mask) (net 17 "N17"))
  (pad 5 thru_hole oval (at 7.62 7.62 180) (size 1.6 1.6) (drill 0.8) (layers *.Cu *.Mask) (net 2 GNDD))
  (pad 1 thru_hole rect (at 0 0 180) (size 1.6 1.6) (drill 0.8) (layers *.Cu *.Mask)))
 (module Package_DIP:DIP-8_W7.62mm (layer F.Cu) (at 172.72 141.605 180)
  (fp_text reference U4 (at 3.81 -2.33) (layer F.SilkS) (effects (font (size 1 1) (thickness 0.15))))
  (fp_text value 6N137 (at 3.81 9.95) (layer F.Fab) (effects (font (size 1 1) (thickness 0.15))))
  (pad 8 thru_hole oval (at 7.62 0 180) (size 1.6 1.6) (drill 0.8) (layers *.Cu *.Mask) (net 1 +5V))
  (pad 4 thru_hole oval (at 0 7.62 180) (size 1.6 1.6) (drill 0.8) (layers *.Cu *.Mask))
  (pad 7 thru_hole oval (at 7.62 2.54 180) (size 1.6 1.6) (drill 0.8) (layers *.Cu *.Mask) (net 1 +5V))
  (pad 3 thru_hole oval (at 0 5.08 180) (size 1.6 1.6) (drill 0.8) (layers *.Cu *.Mask) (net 4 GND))
  (pad 6 thru_hole oval (at 7.62 5.08 180) (size 1.6 1.6) (drill 0.8) (layers *.Cu *.Mask) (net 13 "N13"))
  (pad 2 thru_hole oval (at 0 2.54 180) (size 1.6 1.6) (drill 0.8) (layers *.Cu *.Mask) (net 18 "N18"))
  (pad 5 thru_hole oval (at 7.62 7.62 180) (size 1.6 1.6) (drill 0.8) (layers *.Cu *.Mask) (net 2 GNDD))
  (pad 1 thru_hole rect (at 0 0 180) (size 1.6 1.6) (drill 0.8) (layers *.Cu *.Mask)))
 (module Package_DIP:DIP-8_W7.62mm (layer F.Cu) (at 172.72 128.905 180)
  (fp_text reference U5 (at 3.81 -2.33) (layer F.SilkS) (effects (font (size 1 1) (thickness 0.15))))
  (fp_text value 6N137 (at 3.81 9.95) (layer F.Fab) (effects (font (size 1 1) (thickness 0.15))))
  (pad 1 thru_hole rect (at 0 0 180) (size 1.6 1.6) (drill 0.8) (layers *.Cu *.Mask))
  (pad 5 thru_hole oval (at 7.62 7.62 180) (size 1.6 1.6) (drill 0.8) (layers *.Cu *.Mask) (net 2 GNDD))
  (pad 2 thru_hole oval (at 0 2.54 180) (size 1.6 1.6) (drill 0.8) (layers *.Cu *.Mask) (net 19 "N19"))
  (pad 6 thru_hole oval (at 7.62 5.08 180) (size 1.6 1.6) (drill 0.8) (layers *.Cu *.Mask) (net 14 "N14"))
  (pad 3 thru_hole oval (at 0 5.08 180) (size 1.6 1.6) (drill 0.8) (layers *.Cu *.Mask) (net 4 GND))
  (pad 7 thru_hole oval (at 7.62 2.54 180) (size 1.6 1.6) (drill 0.8) (layers *.Cu *.Mask) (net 1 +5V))
  (pad 4 thru_hole oval (at 0 7.62 180) (size 1.6 1.6) (drill 0.8) (layers *.Cu *.Mask))
  (pad 8 thru_hole oval (at 7.62 0 180) (size 1.6 1.6) (drill 0.8) (layers *.Cu *.Mask) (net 1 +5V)))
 (gr_line (start 210.82 48.26) (end 102.235 48.26) (layer Edge.Cuts) (width 0.05))
 (gr_line (start 210.82 148.59) (end 210.82 48.26) (layer Edge.Cuts) (width 0.05))
 (gr_line (start 102.235 148.59) (end 210.82 148.59) (layer Edge.Cuts) (width 0.05))
 (gr_line (start 102.235 48.26) (end 102.235 148.59) (layer Edge.Cuts) (width 0.05))
 (segment (start 134.62 99.06) (end 127 99.06) (width 1) (layer F.Cu) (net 3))
 (segment (start 134.62 124.46) (end 134.62 99.06) (width 1) (layer F.Cu) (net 3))
 (segment (start 182.99251 119.38) (end 182.35751 120.015) (width 1) (layer F.Cu) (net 5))
 (segment (start 187.96 119.38) (end 182.99251 119.38) (width 1) (layer F.Cu) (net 5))
 (segment (start 183.62751 114.3) (end 182.35751 115.57) (width 1) (layer F.Cu) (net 6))
 (segment (start 187.96 114.3) (end 183.62751 114.3) (width 1) (layer F.Cu) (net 6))
 (segment (start 182.99251 111.76) (end 182.35751 111.125) (width 1) (layer F.Cu) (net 7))
 (segment (start 187.96 111.76) (end 182.99251 111.76) (width 1) (layer F.Cu) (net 7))
 (segment (start 187.96 106.68) (end 182.32751 106.68) (width 1) (layer F.Cu) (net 8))
 (segment (start 184.26251 104.14) (end 182.35751 102.235) (width 1) (layer F.Cu) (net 9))
 (segment (start 187.96 104.14) (end 184.26251 104.14) (width 1) (layer F.Cu) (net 9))
 (segment (start 177.71749 113.665) (end 180.25749 111.125) (width 1) (layer F.Cu) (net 15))
 (segment (start 172.72 113.665) (end 177.71749 113.665) (width 1) (layer F.Cu) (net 15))
 (segment (start 180.25749 101.05646) (end 180.25749 102.235) (width 1) (layer F.Cu) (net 16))
 (segment (start 180.25749 94.677488) (end 180.25749 101.05646) (width 1) (layer F.Cu) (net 16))
 (segment (start 172.72 88.9) (end 174.480002 88.9) (width 1) (layer F.Cu) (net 16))
 (segment (start 174.480002 88.9) (end 180.25749 94.677488) (width 1) (layer F.Cu) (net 16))
 (segment (start 180.22749 106.56749) (end 180.22749 106.68) (width 1) (layer F.Cu) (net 17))
 (segment (start 172.72 101.6) (end 175.26 101.6) (width 1) (layer F.Cu) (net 17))
 (segment (start 175.26 101.6) (end 180.22749 106.56749) (width 1) (layer F.Cu) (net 17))
 (segment (start 180.25749 121.19354) (end 180.25749 120.015) (width 1) (layer F.Cu) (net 18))
 (segment (start 180.25749 132.65888) (end 180.25749 121.19354) (width 1) (layer F.Cu) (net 18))
 (segment (start 172.72 139.065) (end 173.85137 139.065) (width 1) (layer F.Cu) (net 18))
 (segment (start 173.85137 139.065) (end 180.25749 132.65888) (width 1) (layer F.Cu) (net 18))
 (segment (start 173.85137 126.365) (end 175.895 124.32137) (width 1) (layer F.Cu) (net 19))
 (segment (start 172.72 126.365) (end 173.85137 126.365) (width 1) (layer F.Cu) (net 19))
 (segment (start 180.25749 115.68251) (end 180.25749 115.57) (width 1) (layer F.Cu) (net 19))
 (segment (start 175.895 124.32137) (end 175.895 120.045) (width 1) (layer F.Cu) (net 19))
 (segment (start 175.895 120.045) (end 180.25749 115.68251) (width 1) (layer F.Cu) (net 19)))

